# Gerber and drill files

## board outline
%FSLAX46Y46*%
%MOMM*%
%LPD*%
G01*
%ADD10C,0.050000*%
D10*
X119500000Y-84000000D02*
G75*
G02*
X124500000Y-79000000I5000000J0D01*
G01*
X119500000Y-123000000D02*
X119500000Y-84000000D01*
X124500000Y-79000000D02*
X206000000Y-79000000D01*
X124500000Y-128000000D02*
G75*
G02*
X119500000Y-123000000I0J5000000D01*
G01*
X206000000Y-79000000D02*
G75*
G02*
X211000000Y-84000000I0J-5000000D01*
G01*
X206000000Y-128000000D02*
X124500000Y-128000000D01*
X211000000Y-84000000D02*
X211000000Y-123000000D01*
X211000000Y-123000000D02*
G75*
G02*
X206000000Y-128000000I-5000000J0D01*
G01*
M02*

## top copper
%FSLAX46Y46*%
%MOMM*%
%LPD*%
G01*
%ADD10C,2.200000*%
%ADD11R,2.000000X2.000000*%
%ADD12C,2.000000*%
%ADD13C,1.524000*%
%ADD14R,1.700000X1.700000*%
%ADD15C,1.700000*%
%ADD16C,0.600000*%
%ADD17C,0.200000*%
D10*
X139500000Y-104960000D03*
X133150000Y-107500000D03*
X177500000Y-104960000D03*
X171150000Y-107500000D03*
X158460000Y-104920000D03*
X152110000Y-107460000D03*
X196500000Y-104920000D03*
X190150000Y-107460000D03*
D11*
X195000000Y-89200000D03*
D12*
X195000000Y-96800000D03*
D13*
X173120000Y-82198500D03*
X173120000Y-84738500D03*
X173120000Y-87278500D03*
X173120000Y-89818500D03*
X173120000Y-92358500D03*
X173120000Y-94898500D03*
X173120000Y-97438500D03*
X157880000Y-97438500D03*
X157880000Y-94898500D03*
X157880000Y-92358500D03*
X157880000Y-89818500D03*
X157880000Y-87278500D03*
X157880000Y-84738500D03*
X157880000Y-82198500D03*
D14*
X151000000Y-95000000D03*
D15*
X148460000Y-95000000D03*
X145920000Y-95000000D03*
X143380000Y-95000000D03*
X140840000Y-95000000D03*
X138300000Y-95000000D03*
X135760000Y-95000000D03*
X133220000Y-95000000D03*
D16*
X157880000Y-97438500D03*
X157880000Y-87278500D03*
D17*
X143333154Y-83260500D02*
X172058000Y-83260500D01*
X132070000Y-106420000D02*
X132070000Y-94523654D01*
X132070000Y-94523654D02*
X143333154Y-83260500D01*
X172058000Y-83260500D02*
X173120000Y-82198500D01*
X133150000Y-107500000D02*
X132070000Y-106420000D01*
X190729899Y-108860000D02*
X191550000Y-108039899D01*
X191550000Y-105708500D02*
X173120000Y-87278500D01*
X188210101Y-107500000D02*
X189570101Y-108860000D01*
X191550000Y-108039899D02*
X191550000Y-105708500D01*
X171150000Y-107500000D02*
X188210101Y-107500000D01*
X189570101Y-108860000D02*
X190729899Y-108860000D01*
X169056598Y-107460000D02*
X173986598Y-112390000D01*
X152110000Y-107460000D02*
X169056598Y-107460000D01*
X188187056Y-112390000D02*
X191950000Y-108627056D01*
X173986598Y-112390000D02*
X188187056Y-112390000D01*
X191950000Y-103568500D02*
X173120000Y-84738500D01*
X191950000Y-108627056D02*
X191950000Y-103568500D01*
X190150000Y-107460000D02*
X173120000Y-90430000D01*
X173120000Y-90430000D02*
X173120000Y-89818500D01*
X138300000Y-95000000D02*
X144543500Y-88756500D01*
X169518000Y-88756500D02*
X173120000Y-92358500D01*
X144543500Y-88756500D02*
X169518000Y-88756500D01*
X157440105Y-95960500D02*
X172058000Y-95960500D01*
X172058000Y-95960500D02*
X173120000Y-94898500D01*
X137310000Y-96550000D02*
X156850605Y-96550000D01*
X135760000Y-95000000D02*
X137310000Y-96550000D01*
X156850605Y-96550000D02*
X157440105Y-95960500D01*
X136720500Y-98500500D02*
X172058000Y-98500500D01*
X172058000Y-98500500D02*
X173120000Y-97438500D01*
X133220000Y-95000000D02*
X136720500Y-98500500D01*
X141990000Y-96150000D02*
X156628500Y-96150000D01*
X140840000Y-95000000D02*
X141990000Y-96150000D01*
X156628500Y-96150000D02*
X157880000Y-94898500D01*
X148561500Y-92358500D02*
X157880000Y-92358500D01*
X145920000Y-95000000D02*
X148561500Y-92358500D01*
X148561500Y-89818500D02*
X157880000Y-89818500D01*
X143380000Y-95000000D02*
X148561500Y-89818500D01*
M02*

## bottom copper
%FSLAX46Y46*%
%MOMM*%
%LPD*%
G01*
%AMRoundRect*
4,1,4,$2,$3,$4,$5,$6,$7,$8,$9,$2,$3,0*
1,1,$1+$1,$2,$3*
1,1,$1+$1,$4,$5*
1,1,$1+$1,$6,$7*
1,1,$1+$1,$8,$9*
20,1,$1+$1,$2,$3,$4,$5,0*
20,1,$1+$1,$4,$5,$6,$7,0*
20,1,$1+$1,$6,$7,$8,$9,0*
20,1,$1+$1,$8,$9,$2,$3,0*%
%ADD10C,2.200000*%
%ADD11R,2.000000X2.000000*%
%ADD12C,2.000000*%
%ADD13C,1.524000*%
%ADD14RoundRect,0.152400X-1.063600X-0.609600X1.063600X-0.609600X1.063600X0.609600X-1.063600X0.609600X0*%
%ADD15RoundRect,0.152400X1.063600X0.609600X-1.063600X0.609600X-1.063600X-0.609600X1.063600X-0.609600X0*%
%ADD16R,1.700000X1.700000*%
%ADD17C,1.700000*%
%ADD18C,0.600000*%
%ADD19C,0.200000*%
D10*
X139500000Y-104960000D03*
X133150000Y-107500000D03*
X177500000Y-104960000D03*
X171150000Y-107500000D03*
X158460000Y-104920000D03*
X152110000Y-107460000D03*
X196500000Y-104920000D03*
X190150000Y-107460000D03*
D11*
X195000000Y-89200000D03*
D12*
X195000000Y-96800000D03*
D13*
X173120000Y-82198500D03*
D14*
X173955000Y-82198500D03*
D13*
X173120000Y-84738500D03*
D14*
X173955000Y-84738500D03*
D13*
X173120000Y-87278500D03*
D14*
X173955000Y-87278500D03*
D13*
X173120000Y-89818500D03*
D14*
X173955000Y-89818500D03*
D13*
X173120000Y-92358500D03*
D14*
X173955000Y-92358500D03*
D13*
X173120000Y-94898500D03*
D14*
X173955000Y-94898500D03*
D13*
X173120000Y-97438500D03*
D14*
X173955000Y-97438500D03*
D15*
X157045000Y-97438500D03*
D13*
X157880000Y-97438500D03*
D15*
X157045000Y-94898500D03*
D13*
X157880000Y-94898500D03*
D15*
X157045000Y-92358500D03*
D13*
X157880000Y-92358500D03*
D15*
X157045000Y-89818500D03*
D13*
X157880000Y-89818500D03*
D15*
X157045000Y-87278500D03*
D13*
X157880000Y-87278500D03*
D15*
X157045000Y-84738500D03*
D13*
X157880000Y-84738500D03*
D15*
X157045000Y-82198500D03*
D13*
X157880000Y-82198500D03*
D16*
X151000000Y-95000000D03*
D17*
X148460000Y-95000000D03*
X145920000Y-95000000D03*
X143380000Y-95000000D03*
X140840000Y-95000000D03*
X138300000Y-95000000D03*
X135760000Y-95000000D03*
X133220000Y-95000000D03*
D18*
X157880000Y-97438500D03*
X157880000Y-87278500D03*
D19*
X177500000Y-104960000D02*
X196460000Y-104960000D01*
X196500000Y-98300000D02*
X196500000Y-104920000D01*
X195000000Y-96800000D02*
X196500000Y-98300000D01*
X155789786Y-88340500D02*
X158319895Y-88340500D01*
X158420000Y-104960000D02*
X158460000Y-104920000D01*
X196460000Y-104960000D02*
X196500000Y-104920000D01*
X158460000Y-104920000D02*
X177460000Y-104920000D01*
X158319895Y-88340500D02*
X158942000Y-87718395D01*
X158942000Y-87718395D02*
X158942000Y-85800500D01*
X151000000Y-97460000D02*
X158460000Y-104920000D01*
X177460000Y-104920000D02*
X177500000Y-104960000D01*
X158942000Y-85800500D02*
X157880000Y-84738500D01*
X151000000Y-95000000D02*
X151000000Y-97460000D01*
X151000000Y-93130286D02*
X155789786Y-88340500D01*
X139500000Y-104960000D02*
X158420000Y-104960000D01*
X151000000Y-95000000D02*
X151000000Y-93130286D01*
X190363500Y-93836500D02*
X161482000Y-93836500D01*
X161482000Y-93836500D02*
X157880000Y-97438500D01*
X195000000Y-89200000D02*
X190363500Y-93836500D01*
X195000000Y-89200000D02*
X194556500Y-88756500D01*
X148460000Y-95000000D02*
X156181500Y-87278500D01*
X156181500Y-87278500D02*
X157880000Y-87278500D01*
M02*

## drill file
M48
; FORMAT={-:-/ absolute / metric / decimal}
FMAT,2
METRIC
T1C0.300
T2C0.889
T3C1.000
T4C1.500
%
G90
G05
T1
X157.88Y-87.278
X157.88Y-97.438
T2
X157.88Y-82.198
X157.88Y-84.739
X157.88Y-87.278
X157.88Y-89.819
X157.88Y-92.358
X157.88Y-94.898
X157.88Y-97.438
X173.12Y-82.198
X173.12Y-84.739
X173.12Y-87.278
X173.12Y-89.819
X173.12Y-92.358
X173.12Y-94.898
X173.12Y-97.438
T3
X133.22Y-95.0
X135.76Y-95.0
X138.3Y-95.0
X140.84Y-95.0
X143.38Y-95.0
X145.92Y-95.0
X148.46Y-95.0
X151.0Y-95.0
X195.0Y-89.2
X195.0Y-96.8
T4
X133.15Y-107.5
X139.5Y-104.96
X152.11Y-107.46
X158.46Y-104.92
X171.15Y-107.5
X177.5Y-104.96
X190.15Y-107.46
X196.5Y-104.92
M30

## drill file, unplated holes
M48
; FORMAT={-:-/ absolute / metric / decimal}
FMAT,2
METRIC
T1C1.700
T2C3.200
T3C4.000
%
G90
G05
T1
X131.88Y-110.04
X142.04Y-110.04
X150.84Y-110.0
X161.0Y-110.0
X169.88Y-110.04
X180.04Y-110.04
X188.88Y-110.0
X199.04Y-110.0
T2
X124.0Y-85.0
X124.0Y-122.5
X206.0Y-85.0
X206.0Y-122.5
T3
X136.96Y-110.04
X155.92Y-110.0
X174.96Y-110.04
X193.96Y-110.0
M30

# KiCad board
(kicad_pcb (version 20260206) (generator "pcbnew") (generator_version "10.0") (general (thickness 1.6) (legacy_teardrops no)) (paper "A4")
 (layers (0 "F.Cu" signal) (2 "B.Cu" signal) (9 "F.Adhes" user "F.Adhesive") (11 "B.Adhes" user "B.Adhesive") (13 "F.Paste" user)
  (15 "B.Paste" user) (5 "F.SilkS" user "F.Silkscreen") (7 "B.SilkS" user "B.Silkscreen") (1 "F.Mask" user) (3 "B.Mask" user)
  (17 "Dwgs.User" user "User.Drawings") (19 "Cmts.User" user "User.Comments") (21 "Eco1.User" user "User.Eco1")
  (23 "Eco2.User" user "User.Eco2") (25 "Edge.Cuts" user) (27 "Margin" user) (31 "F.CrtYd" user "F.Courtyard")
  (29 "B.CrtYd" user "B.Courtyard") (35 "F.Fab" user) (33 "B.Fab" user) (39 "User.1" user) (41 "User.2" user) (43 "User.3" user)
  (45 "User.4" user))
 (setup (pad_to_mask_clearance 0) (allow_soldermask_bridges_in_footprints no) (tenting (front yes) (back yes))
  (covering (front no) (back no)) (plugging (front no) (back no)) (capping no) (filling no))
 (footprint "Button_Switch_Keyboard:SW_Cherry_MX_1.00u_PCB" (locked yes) (layer "F.Cu") (at 139.5 104.96)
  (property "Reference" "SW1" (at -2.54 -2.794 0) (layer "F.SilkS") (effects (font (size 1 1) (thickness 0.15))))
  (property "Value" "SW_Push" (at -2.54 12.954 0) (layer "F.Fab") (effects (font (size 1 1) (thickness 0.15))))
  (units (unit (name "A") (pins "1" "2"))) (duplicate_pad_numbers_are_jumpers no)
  (pad "" np_thru_hole circle (at -7.62 5.08) (size 1.7 1.7) (drill 1.7) (layers "*.Cu" "*.Mask"))
  (pad "" np_thru_hole circle (at -2.54 5.08) (size 4 4) (drill 4) (layers "*.Cu" "*.Mask"))
  (pad "" np_thru_hole circle (at 2.54 5.08) (size 1.7 1.7) (drill 1.7) (layers "*.Cu" "*.Mask"))
  (pad "1" thru_hole circle (at 0 0) (size 2.2 2.2) (drill 1.5) (layers "*.Cu" "*.Mask") (remove_unused_layers no) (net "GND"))
  (pad "2" thru_hole circle (at -6.35 2.54) (size 2.2 2.2) (drill 1.5) (layers "*.Cu" "*.Mask") (remove_unused_layers no)
   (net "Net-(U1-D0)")))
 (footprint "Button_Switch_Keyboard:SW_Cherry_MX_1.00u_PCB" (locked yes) (layer "F.Cu") (at 177.5 104.96)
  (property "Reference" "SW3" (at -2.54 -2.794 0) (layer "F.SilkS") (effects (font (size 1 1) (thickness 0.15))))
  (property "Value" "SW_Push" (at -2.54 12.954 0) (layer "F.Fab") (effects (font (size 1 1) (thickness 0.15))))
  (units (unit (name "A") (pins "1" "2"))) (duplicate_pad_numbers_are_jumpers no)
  (pad "" np_thru_hole circle (at -7.62 5.08) (size 1.7 1.7) (drill 1.7) (layers "*.Cu" "*.Mask"))
  (pad "" np_thru_hole circle (at -2.54 5.08) (size 4 4) (drill 4) (layers "*.Cu" "*.Mask"))
  (pad "" np_thru_hole circle (at 2.54 5.08) (size 1.7 1.7) (drill 1.7) (layers "*.Cu" "*.Mask"))
  (pad "1" thru_hole circle (at 0 0) (size 2.2 2.2) (drill 1.5) (layers "*.Cu" "*.Mask") (remove_unused_layers no) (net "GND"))
  (pad "2" thru_hole circle (at -6.35 2.54) (size 2.2 2.2) (drill 1.5) (layers "*.Cu" "*.Mask") (remove_unused_layers no)
   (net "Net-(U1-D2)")))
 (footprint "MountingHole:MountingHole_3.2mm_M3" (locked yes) (layer "F.Cu") (at 206 85)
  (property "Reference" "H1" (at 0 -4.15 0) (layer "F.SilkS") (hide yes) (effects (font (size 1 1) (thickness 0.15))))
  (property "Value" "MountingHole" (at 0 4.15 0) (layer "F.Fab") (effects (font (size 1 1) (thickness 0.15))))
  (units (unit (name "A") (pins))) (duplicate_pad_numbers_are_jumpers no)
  (pad "" np_thru_hole circle (at 0 0) (size 3.2 3.2) (drill 3.2) (layers "*.Cu" "*.Mask")))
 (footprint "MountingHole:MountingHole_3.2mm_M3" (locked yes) (layer "F.Cu") (at 206 122.5)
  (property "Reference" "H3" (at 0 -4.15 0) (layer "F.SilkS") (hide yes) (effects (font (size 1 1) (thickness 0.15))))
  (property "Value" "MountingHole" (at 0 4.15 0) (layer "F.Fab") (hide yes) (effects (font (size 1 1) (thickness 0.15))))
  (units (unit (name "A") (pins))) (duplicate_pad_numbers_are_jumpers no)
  (pad "" np_thru_hole circle (at 0 0) (size 3.2 3.2) (drill 3.2) (layers "*.Cu" "*.Mask")))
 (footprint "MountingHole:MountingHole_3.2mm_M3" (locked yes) (layer "F.Cu") (at 124 122.5)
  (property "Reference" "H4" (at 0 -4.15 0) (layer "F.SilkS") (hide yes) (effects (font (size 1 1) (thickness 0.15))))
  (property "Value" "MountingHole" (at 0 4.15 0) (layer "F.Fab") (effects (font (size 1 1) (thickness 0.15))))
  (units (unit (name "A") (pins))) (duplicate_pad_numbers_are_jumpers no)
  (pad "" np_thru_hole circle (at 0 0) (size 3.2 3.2) (drill 3.2) (layers "*.Cu" "*.Mask")))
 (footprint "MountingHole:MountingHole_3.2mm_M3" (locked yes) (layer "F.Cu") (at 124 85)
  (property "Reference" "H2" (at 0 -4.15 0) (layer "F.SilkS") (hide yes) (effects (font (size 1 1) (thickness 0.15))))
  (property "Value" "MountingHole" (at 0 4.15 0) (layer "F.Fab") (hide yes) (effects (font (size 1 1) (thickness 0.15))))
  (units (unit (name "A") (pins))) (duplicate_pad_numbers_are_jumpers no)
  (pad "" np_thru_hole circle (at 0 0) (size 3.2 3.2) (drill 3.2) (layers "*.Cu" "*.Mask")))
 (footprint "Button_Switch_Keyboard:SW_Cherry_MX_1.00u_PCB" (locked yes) (layer "F.Cu") (at 158.46 104.92)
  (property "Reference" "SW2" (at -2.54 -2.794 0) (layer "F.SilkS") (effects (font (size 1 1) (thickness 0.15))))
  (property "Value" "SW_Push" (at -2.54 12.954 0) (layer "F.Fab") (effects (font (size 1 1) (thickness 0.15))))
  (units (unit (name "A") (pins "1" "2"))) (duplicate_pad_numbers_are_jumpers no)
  (pad "" np_thru_hole circle (at -7.62 5.08) (size 1.7 1.7) (drill 1.7) (layers "*.Cu" "*.Mask"))
  (pad "" np_thru_hole circle (at -2.54 5.08) (size 4 4) (drill 4) (layers "*.Cu" "*.Mask"))
  (pad "" np_thru_hole circle (at 2.54 5.08) (size 1.7 1.7) (drill 1.7) (layers "*.Cu" "*.Mask"))
  (pad "1" thru_hole circle (at 0 0) (size 2.2 2.2) (drill 1.5) (layers "*.Cu" "*.Mask") (remove_unused_layers no) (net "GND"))
  (pad "2" thru_hole circle (at -6.35 2.54) (size 2.2 2.2) (drill 1.5) (layers "*.Cu" "*.Mask") (remove_unused_layers no)
   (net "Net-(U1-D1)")))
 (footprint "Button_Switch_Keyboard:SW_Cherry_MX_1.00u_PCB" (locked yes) (layer "F.Cu") (at 196.5 104.92)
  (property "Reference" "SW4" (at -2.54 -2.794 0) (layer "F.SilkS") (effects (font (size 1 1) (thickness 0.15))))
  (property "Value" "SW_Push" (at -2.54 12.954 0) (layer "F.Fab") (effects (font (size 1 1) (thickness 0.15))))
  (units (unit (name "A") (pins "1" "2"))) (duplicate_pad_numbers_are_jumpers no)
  (pad "" np_thru_hole circle (at -7.62 5.08) (size 1.7 1.7) (drill 1.7) (layers "*.Cu" "*.Mask"))
  (pad "" np_thru_hole circle (at -2.54 5.08) (size 4 4) (drill 4) (layers "*.Cu" "*.Mask"))
  (pad "" np_thru_hole circle (at 2.54 5.08) (size 1.7 1.7) (drill 1.7) (layers "*.Cu" "*.Mask"))
  (pad "1" thru_hole circle (at 0 0) (size 2.2 2.2) (drill 1.5) (layers "*.Cu" "*.Mask") (remove_unused_layers no) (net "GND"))
  (pad "2" thru_hole circle (at -6.35 2.54) (size 2.2 2.2) (drill 1.5) (layers "*.Cu" "*.Mask") (remove_unused_layers no)
   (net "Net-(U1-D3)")))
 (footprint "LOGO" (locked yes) (layer "F.Cu") (at 187.4 86.2)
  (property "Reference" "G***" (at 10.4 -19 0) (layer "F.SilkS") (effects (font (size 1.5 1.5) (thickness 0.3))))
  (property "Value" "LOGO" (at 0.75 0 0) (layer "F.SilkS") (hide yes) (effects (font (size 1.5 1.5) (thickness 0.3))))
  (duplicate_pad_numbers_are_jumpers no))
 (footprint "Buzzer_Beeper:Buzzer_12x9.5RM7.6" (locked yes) (layer "B.Cu") (at 195 89.2 -90)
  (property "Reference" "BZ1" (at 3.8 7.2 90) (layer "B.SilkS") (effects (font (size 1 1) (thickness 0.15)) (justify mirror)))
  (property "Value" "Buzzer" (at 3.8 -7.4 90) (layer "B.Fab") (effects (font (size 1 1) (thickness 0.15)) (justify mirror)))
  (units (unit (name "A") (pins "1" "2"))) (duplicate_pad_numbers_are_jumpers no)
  (pad "1" thru_hole rect (at 0 0 270) (size 2 2) (drill 1) (layers "*.Cu" "*.Mask") (remove_unused_layers no) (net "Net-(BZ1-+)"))
  (pad "2" thru_hole circle (at 7.6 0 270) (size 2 2) (drill 1) (layers "*.Cu" "*.Mask") (remove_unused_layers no) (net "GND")))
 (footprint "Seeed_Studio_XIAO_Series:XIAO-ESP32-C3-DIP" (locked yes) (layer "B.Cu") (at 165.5 89.8185 90)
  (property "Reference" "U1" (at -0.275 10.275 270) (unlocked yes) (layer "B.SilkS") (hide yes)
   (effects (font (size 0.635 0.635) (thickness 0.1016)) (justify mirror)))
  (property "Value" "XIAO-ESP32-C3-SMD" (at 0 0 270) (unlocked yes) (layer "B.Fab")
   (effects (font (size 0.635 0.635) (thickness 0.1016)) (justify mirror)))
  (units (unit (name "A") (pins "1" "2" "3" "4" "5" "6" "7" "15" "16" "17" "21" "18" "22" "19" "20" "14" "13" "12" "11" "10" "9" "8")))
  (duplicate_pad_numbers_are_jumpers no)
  (pad "1" thru_hole circle (at 7.62 7.62) (size 1.524 1.524) (drill 0.889) (layers "*.Cu" "*.Mask") (remove_unused_layers no)
   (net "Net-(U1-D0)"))
  (pad "1" smd roundrect (at 7.62 8.455) (size 2.432 1.524) (layers "B.Cu" "B.Mask") (roundrect_rratio 0.1) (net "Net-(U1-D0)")
   (thermal_bridge_angle 45))
  (pad "2" thru_hole circle (at 5.08 7.62) (size 1.524 1.524) (drill 0.889) (layers "*.Cu" "*.Mask") (remove_unused_layers no)
   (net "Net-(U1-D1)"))
  (pad "2" smd roundrect (at 5.08 8.455) (size 2.432 1.524) (layers "B.Cu" "B.Mask") (roundrect_rratio 0.1) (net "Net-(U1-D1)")
   (thermal_bridge_angle 45))
  (pad "3" thru_hole circle (at 2.54 7.62) (size 1.524 1.524) (drill 0.889) (layers "*.Cu" "*.Mask") (remove_unused_layers no)
   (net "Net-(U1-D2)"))
  (pad "3" smd roundrect (at 2.54 8.455) (size 2.432 1.524) (layers "B.Cu" "B.Mask") (roundrect_rratio 0.1) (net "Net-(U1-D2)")
   (thermal_bridge_angle 45))
  (pad "4" thru_hole circle (at 0 7.62) (size 1.524 1.524) (drill 0.889) (layers "*.Cu" "*.Mask") (remove_unused_layers no)
   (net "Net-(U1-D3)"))
  (pad "4" smd roundrect (at 0 8.455) (size 2.432 1.524) (layers "B.Cu" "B.Mask") (roundrect_rratio 0.1) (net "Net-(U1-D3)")
   (thermal_bridge_angle 45))
  (pad "5" thru_hole circle (at -2.54 7.62) (size 1.524 1.524) (drill 0.889) (layers "*.Cu" "*.Mask") (remove_unused_layers no)
   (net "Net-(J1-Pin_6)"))
  (pad "5" smd roundrect (at -2.54 8.455) (size 2.432 1.524) (layers "B.Cu" "B.Mask") (roundrect_rratio 0.1) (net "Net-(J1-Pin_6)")
   (thermal_bridge_angle 45))
  (pad "6" thru_hole circle (at -5.08 7.62) (size 1.524 1.524) (drill 0.889) (layers "*.Cu" "*.Mask") (remove_unused_layers no)
   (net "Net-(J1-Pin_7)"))
  (pad "6" smd roundrect (at -5.08 8.455) (size 2.432 1.524) (layers "B.Cu" "B.Mask") (roundrect_rratio 0.1) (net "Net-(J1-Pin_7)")
   (thermal_bridge_angle 45))
  (pad "7" thru_hole circle (at -7.62 7.62) (size 1.524 1.524) (drill 0.889) (layers "*.Cu" "*.Mask") (remove_unused_layers no)
   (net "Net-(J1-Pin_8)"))
  (pad "7" smd roundrect (at -7.62 8.455) (size 2.432 1.524) (layers "B.Cu" "B.Mask") (roundrect_rratio 0.1) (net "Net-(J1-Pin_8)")
   (thermal_bridge_angle 45))
  (pad "8" smd roundrect (at -7.62 -8.455 180) (size 2.432 1.524) (layers "B.Cu" "B.Mask") (roundrect_rratio 0.1) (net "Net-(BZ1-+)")
   (thermal_bridge_angle 45))
  (pad "8" thru_hole circle (at -7.62 -7.62 180) (size 1.524 1.524) (drill 0.889) (layers "*.Cu" "*.Mask") (remove_unused_layers no)
   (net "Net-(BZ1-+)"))
  (pad "9" smd roundrect (at -5.08 -8.455 180) (size 2.432 1.524) (layers "B.Cu" "B.Mask") (roundrect_rratio 0.1) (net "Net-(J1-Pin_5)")
   (thermal_bridge_angle 45))
  (pad "9" thru_hole circle (at -5.08 -7.62 180) (size 1.524 1.524) (drill 0.889) (layers "*.Cu" "*.Mask") (remove_unused_layers no)
   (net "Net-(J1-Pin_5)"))
  (pad "10" smd roundrect (at -2.54 -8.455 180) (size 2.432 1.524) (layers "B.Cu" "B.Mask") (roundrect_rratio 0.1) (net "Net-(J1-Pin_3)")
   (thermal_bridge_angle 45))
  (pad "10" thru_hole circle (at -2.54 -7.62 180) (size 1.524 1.524) (drill 0.889) (layers "*.Cu" "*.Mask") (remove_unused_layers no)
   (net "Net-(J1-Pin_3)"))
  (pad "11" smd roundrect (at 0 -8.455 180) (size 2.432 1.524) (layers "B.Cu" "B.Mask") (roundrect_rratio 0.1) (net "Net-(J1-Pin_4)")
   (thermal_bridge_angle 45))
  (pad "11" thru_hole circle (at 0 -7.62 180) (size 1.524 1.524) (drill 0.889) (layers "*.Cu" "*.Mask") (remove_unused_layers no)
   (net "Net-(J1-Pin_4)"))
  (pad "12" smd roundrect (at 2.54 -8.455 180) (size 2.432 1.524) (layers "B.Cu" "B.Mask") (roundrect_rratio 0.1) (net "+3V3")
   (thermal_bridge_angle 45))
  (pad "12" thru_hole circle (at 2.54 -7.62 180) (size 1.524 1.524) (drill 0.889) (layers "*.Cu" "*.Mask") (remove_unused_layers no)
   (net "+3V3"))
  (pad "13" smd roundrect (at 5.08 -8.455 180) (size 2.432 1.524) (layers "B.Cu" "B.Mask") (roundrect_rratio 0.1) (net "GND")
   (thermal_bridge_angle 45))
  (pad "13" thru_hole circle (at 5.08 -7.62 180) (size 1.524 1.524) (drill 0.889) (layers "*.Cu" "*.Mask") (remove_unused_layers no)
   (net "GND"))
  (pad "14" smd roundrect (at 7.62 -8.455 180) (size 2.432 1.524) (layers "B.Cu" "B.Mask") (roundrect_rratio 0.1)
   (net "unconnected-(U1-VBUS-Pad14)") (thermal_bridge_angle 45))
  (pad "14" thru_hole circle (at 7.62 -7.62 180) (size 1.524 1.524) (drill 0.889) (layers "*.Cu" "*.Mask") (remove_unused_layers no)
   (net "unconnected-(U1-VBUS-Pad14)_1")))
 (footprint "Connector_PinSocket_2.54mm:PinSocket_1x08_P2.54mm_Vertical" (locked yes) (layer "B.Cu") (at 151 95 90)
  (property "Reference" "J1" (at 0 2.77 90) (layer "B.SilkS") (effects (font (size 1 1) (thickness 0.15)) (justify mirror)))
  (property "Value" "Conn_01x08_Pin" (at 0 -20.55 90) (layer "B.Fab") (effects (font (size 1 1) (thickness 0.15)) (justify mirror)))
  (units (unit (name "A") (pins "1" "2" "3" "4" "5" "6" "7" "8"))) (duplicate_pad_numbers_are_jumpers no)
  (pad "1" thru_hole rect (at 0 0 90) (size 1.7 1.7) (drill 1) (layers "*.Cu" "*.Mask") (remove_unused_layers no) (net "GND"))
  (pad "2" thru_hole circle (at 0 -2.54 90) (size 1.7 1.7) (drill 1) (layers "*.Cu" "*.Mask") (remove_unused_layers no) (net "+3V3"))
  (pad "3" thru_hole circle (at 0 -5.08 90) (size 1.7 1.7) (drill 1) (layers "*.Cu" "*.Mask") (remove_unused_layers no)
   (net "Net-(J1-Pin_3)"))
  (pad "4" thru_hole circle (at 0 -7.62 90) (size 1.7 1.7) (drill 1) (layers "*.Cu" "*.Mask") (remove_unused_layers no)
   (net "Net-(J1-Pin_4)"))
  (pad "5" thru_hole circle (at 0 -10.16 90) (size 1.7 1.7) (drill 1) (layers "*.Cu" "*.Mask") (remove_unused_layers no)
   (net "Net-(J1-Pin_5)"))
  (pad "6" thru_hole circle (at 0 -12.7 90) (size 1.7 1.7) (drill 1) (layers "*.Cu" "*.Mask") (remove_unused_layers no)
   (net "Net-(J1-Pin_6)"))
  (pad "7" thru_hole circle (at 0 -15.24 90) (size 1.7 1.7) (drill 1) (layers "*.Cu" "*.Mask") (remove_unused_layers no)
   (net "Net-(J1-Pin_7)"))
  (pad "8" thru_hole circle (at 0 -17.78 90) (size 1.7 1.7) (drill 1) (layers "*.Cu" "*.Mask") (remove_unused_layers no)
   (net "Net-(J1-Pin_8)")))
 (gr_arc (start 119.5 84) (mid 120.964466 80.464466) (end 124.5 79) (stroke (width 0.05) (type default)) (locked yes) (layer "Edge.Cuts"))
 (gr_line (start 119.5 123) (end 119.5 84) (stroke (width 0.05) (type default)) (locked yes) (layer "Edge.Cuts"))
 (gr_line (start 124.5 79) (end 206 79) (stroke (width 0.05) (type default)) (locked yes) (layer "Edge.Cuts"))
 (gr_arc (start 124.5 128) (mid 120.964466 126.535534) (end 119.5 123) (stroke (width 0.05) (type default)) (locked yes) (layer "Edge.Cuts"))
 (gr_arc (start 206 79) (mid 209.535534 80.464466) (end 211 84) (stroke (width 0.05) (type default)) (locked yes) (layer "Edge.Cuts"))
 (gr_line (start 206 128) (end 124.5 128) (stroke (width 0.05) (type default)) (locked yes) (layer "Edge.Cuts"))
 (gr_line (start 211 84) (end 211 123) (stroke (width 0.05) (type default)) (locked yes) (layer "Edge.Cuts"))
 (gr_arc (start 211 123) (mid 209.535534 126.535534) (end 206 128) (stroke (width 0.05) (type default)) (locked yes) (layer "Edge.Cuts"))
 (segment (start 177.5 104.96) (end 196.46 104.96) (width 0.2) (locked yes) (layer "B.Cu") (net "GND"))
 (segment (start 196.5 98.3) (end 196.5 104.92) (width 0.2) (locked yes) (layer "B.Cu") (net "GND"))
 (segment (start 195 96.8) (end 196.5 98.3) (width 0.2) (locked yes) (layer "B.Cu") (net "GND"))
 (segment (start 155.789786 88.3405) (end 158.319895 88.3405) (width 0.2) (locked yes) (layer "B.Cu") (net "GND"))
 (segment (start 158.42 104.96) (end 158.46 104.92) (width 0.2) (locked yes) (layer "B.Cu") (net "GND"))
 (segment (start 196.46 104.96) (end 196.5 104.92) (width 0.2) (locked yes) (layer "B.Cu") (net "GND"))
 (segment (start 158.46 104.92) (end 177.46 104.92) (width 0.2) (locked yes) (layer "B.Cu") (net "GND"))
 (segment (start 158.319895 88.3405) (end 158.942 87.718395) (width 0.2) (locked yes) (layer "B.Cu") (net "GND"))
 (segment (start 158.942 87.718395) (end 158.942 85.8005) (width 0.2) (locked yes) (layer "B.Cu") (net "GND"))
 (segment (start 151 97.46) (end 158.46 104.92) (width 0.2) (locked yes) (layer "B.Cu") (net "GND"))
 (segment (start 177.46 104.92) (end 177.5 104.96) (width 0.2) (locked yes) (layer "B.Cu") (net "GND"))
 (segment (start 158.942 85.8005) (end 157.88 84.7385) (width 0.2) (locked yes) (layer "B.Cu") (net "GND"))
 (segment (start 151 95) (end 151 97.46) (width 0.2) (locked yes) (layer "B.Cu") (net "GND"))
 (segment (start 151 93.130286) (end 155.789786 88.3405) (width 0.2) (locked yes) (layer "B.Cu") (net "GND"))
 (segment (start 139.5 104.96) (end 158.42 104.96) (width 0.2) (locked yes) (layer "B.Cu") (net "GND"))
 (segment (start 151 95) (end 151 93.130286) (width 0.2) (locked yes) (layer "B.Cu") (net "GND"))
 (segment (start 143.333154 83.2605) (end 172.058 83.2605) (width 0.2) (locked yes) (layer "F.Cu") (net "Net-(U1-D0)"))
 (segment (start 132.07 106.42) (end 132.07 94.523654) (width 0.2) (locked yes) (layer "F.Cu") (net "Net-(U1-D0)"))
 (segment (start 132.07 94.523654) (end 143.333154 83.2605) (width 0.2) (locked yes) (layer "F.Cu") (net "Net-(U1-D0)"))
 (segment (start 172.058 83.2605) (end 173.12 82.1985) (width 0.2) (locked yes) (layer "F.Cu") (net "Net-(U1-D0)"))
 (segment (start 133.15 107.5) (end 132.07 106.42) (width 0.2) (locked yes) (layer "F.Cu") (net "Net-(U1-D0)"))
 (segment (start 190.729899 108.86) (end 191.55 108.039899) (width 0.2) (locked yes) (layer "F.Cu") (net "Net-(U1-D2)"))
 (segment (start 191.55 105.7085) (end 173.12 87.2785) (width 0.2) (locked yes) (layer "F.Cu") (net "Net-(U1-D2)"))
 (segment (start 188.210101 107.5) (end 189.570101 108.86) (width 0.2) (locked yes) (layer "F.Cu") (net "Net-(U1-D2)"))
 (segment (start 191.55 108.039899) (end 191.55 105.7085) (width 0.2) (locked yes) (layer "F.Cu") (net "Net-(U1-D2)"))
 (segment (start 171.15 107.5) (end 188.210101 107.5) (width 0.2) (locked yes) (layer "F.Cu") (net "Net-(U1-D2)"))
 (segment (start 189.570101 108.86) (end 190.729899 108.86) (width 0.2) (locked yes) (layer "F.Cu") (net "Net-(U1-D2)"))
 (segment (start 169.056598 107.46) (end 173.986598 112.39) (width 0.2) (locked yes) (layer "F.Cu") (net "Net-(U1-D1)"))
 (segment (start 152.11 107.46) (end 169.056598 107.46) (width 0.2) (locked yes) (layer "F.Cu") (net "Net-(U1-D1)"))
 (segment (start 188.187056 112.39) (end 191.95 108.627056) (width 0.2) (locked yes) (layer "F.Cu") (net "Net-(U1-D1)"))
 (segment (start 173.986598 112.39) (end 188.187056 112.39) (width 0.2) (locked yes) (layer "F.Cu") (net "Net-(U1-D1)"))
 (segment (start 191.95 103.5685) (end 173.12 84.7385) (width 0.2) (locked yes) (layer "F.Cu") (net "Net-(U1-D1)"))
 (segment (start 191.95 108.627056) (end 191.95 103.5685) (width 0.2) (locked yes) (layer "F.Cu") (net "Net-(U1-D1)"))
 (segment (start 190.15 107.46) (end 173.12 90.43) (width 0.2) (locked yes) (layer "F.Cu") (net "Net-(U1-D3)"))
 (segment (start 173.12 90.43) (end 173.12 89.8185) (width 0.2) (locked yes) (layer "F.Cu") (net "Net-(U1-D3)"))
 (via (at 157.88 97.4385) (size 0.6) (drill 0.3) (layers "F.Cu" "B.Cu") (locked yes) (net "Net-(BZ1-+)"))
 (segment (start 190.3635 93.8365) (end 161.482 93.8365) (width 0.2) (locked yes) (layer "B.Cu") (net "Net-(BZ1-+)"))
 (segment (start 161.482 93.8365) (end 157.88 97.4385) (width 0.2) (locked yes) (layer "B.Cu") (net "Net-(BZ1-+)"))
 (segment (start 195 89.2) (end 190.3635 93.8365) (width 0.2) (locked yes) (layer "B.Cu") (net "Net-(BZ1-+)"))
 (segment (start 195 89.2) (end 194.5565 88.7565) (width 0.2) (locked yes) (layer "B.Cu") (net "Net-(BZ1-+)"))
 (segment (start 138.3 95) (end 144.5435 88.7565) (width 0.2) (locked yes) (layer "F.Cu") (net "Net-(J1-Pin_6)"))
 (segment (start 169.518 88.7565) (end 173.12 92.3585) (width 0.2) (locked yes) (layer "F.Cu") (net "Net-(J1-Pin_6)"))
 (segment (start 144.5435 88.7565) (end 169.518 88.7565) (width 0.2) (locked yes) (layer "F.Cu") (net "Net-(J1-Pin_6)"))
 (segment (start 157.440105 95.9605) (end 172.058 95.9605) (width 0.2) (locked yes) (layer "F.Cu") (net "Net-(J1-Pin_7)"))
 (segment (start 172.058 95.9605) (end 173.12 94.8985) (width 0.2) (locked yes) (layer "F.Cu") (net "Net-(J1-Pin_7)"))
 (segment (start 137.31 96.55) (end 156.850605 96.55) (width 0.2) (locked yes) (layer "F.Cu") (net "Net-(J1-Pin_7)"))
 (segment (start 135.76 95) (end 137.31 96.55) (width 0.2) (locked yes) (layer "F.Cu") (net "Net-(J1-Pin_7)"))
 (segment (start 156.850605 96.55) (end 157.440105 95.9605) (width 0.2) (locked yes) (layer "F.Cu") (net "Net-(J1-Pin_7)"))
 (segment (start 136.7205 98.5005) (end 172.058 98.5005) (width 0.2) (locked yes) (layer "F.Cu") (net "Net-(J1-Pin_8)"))
 (segment (start 172.058 98.5005) (end 173.12 97.4385) (width 0.2) (locked yes) (layer "F.Cu") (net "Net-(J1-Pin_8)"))
 (segment (start 133.22 95) (end 136.7205 98.5005) (width 0.2) (locked yes) (layer "F.Cu") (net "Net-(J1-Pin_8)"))
 (segment (start 141.99 96.15) (end 156.6285 96.15) (width 0.2) (locked yes) (layer "F.Cu") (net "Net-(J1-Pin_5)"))
 (segment (start 140.84 95) (end 141.99 96.15) (width 0.2) (locked yes) (layer "F.Cu") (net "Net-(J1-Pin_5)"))
 (segment (start 156.6285 96.15) (end 157.88 94.8985) (width 0.2) (locked yes) (layer "F.Cu") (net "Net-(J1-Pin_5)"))
 (segment (start 148.5615 92.3585) (end 157.88 92.3585) (width 0.2) (locked yes) (layer "F.Cu") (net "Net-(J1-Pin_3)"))
 (segment (start 145.92 95) (end 148.5615 92.3585) (width 0.2) (locked yes) (layer "F.Cu") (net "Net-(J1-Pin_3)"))
 (segment (start 148.5615 89.8185) (end 157.88 89.8185) (width 0.2) (locked yes) (layer "F.Cu") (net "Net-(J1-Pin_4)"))
 (segment (start 143.38 95) (end 148.5615 89.8185) (width 0.2) (locked yes) (layer "F.Cu") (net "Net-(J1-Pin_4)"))
 (via (at 157.88 87.2785) (size 0.6) (drill 0.3) (layers "F.Cu" "B.Cu") (locked yes) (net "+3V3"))
 (segment (start 148.46 95) (end 156.1815 87.2785) (width 0.2) (locked yes) (layer "B.Cu") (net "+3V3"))
 (segment (start 156.1815 87.2785) (end 157.88 87.2785) (width 0.2) (locked yes) (layer "B.Cu") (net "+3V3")))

